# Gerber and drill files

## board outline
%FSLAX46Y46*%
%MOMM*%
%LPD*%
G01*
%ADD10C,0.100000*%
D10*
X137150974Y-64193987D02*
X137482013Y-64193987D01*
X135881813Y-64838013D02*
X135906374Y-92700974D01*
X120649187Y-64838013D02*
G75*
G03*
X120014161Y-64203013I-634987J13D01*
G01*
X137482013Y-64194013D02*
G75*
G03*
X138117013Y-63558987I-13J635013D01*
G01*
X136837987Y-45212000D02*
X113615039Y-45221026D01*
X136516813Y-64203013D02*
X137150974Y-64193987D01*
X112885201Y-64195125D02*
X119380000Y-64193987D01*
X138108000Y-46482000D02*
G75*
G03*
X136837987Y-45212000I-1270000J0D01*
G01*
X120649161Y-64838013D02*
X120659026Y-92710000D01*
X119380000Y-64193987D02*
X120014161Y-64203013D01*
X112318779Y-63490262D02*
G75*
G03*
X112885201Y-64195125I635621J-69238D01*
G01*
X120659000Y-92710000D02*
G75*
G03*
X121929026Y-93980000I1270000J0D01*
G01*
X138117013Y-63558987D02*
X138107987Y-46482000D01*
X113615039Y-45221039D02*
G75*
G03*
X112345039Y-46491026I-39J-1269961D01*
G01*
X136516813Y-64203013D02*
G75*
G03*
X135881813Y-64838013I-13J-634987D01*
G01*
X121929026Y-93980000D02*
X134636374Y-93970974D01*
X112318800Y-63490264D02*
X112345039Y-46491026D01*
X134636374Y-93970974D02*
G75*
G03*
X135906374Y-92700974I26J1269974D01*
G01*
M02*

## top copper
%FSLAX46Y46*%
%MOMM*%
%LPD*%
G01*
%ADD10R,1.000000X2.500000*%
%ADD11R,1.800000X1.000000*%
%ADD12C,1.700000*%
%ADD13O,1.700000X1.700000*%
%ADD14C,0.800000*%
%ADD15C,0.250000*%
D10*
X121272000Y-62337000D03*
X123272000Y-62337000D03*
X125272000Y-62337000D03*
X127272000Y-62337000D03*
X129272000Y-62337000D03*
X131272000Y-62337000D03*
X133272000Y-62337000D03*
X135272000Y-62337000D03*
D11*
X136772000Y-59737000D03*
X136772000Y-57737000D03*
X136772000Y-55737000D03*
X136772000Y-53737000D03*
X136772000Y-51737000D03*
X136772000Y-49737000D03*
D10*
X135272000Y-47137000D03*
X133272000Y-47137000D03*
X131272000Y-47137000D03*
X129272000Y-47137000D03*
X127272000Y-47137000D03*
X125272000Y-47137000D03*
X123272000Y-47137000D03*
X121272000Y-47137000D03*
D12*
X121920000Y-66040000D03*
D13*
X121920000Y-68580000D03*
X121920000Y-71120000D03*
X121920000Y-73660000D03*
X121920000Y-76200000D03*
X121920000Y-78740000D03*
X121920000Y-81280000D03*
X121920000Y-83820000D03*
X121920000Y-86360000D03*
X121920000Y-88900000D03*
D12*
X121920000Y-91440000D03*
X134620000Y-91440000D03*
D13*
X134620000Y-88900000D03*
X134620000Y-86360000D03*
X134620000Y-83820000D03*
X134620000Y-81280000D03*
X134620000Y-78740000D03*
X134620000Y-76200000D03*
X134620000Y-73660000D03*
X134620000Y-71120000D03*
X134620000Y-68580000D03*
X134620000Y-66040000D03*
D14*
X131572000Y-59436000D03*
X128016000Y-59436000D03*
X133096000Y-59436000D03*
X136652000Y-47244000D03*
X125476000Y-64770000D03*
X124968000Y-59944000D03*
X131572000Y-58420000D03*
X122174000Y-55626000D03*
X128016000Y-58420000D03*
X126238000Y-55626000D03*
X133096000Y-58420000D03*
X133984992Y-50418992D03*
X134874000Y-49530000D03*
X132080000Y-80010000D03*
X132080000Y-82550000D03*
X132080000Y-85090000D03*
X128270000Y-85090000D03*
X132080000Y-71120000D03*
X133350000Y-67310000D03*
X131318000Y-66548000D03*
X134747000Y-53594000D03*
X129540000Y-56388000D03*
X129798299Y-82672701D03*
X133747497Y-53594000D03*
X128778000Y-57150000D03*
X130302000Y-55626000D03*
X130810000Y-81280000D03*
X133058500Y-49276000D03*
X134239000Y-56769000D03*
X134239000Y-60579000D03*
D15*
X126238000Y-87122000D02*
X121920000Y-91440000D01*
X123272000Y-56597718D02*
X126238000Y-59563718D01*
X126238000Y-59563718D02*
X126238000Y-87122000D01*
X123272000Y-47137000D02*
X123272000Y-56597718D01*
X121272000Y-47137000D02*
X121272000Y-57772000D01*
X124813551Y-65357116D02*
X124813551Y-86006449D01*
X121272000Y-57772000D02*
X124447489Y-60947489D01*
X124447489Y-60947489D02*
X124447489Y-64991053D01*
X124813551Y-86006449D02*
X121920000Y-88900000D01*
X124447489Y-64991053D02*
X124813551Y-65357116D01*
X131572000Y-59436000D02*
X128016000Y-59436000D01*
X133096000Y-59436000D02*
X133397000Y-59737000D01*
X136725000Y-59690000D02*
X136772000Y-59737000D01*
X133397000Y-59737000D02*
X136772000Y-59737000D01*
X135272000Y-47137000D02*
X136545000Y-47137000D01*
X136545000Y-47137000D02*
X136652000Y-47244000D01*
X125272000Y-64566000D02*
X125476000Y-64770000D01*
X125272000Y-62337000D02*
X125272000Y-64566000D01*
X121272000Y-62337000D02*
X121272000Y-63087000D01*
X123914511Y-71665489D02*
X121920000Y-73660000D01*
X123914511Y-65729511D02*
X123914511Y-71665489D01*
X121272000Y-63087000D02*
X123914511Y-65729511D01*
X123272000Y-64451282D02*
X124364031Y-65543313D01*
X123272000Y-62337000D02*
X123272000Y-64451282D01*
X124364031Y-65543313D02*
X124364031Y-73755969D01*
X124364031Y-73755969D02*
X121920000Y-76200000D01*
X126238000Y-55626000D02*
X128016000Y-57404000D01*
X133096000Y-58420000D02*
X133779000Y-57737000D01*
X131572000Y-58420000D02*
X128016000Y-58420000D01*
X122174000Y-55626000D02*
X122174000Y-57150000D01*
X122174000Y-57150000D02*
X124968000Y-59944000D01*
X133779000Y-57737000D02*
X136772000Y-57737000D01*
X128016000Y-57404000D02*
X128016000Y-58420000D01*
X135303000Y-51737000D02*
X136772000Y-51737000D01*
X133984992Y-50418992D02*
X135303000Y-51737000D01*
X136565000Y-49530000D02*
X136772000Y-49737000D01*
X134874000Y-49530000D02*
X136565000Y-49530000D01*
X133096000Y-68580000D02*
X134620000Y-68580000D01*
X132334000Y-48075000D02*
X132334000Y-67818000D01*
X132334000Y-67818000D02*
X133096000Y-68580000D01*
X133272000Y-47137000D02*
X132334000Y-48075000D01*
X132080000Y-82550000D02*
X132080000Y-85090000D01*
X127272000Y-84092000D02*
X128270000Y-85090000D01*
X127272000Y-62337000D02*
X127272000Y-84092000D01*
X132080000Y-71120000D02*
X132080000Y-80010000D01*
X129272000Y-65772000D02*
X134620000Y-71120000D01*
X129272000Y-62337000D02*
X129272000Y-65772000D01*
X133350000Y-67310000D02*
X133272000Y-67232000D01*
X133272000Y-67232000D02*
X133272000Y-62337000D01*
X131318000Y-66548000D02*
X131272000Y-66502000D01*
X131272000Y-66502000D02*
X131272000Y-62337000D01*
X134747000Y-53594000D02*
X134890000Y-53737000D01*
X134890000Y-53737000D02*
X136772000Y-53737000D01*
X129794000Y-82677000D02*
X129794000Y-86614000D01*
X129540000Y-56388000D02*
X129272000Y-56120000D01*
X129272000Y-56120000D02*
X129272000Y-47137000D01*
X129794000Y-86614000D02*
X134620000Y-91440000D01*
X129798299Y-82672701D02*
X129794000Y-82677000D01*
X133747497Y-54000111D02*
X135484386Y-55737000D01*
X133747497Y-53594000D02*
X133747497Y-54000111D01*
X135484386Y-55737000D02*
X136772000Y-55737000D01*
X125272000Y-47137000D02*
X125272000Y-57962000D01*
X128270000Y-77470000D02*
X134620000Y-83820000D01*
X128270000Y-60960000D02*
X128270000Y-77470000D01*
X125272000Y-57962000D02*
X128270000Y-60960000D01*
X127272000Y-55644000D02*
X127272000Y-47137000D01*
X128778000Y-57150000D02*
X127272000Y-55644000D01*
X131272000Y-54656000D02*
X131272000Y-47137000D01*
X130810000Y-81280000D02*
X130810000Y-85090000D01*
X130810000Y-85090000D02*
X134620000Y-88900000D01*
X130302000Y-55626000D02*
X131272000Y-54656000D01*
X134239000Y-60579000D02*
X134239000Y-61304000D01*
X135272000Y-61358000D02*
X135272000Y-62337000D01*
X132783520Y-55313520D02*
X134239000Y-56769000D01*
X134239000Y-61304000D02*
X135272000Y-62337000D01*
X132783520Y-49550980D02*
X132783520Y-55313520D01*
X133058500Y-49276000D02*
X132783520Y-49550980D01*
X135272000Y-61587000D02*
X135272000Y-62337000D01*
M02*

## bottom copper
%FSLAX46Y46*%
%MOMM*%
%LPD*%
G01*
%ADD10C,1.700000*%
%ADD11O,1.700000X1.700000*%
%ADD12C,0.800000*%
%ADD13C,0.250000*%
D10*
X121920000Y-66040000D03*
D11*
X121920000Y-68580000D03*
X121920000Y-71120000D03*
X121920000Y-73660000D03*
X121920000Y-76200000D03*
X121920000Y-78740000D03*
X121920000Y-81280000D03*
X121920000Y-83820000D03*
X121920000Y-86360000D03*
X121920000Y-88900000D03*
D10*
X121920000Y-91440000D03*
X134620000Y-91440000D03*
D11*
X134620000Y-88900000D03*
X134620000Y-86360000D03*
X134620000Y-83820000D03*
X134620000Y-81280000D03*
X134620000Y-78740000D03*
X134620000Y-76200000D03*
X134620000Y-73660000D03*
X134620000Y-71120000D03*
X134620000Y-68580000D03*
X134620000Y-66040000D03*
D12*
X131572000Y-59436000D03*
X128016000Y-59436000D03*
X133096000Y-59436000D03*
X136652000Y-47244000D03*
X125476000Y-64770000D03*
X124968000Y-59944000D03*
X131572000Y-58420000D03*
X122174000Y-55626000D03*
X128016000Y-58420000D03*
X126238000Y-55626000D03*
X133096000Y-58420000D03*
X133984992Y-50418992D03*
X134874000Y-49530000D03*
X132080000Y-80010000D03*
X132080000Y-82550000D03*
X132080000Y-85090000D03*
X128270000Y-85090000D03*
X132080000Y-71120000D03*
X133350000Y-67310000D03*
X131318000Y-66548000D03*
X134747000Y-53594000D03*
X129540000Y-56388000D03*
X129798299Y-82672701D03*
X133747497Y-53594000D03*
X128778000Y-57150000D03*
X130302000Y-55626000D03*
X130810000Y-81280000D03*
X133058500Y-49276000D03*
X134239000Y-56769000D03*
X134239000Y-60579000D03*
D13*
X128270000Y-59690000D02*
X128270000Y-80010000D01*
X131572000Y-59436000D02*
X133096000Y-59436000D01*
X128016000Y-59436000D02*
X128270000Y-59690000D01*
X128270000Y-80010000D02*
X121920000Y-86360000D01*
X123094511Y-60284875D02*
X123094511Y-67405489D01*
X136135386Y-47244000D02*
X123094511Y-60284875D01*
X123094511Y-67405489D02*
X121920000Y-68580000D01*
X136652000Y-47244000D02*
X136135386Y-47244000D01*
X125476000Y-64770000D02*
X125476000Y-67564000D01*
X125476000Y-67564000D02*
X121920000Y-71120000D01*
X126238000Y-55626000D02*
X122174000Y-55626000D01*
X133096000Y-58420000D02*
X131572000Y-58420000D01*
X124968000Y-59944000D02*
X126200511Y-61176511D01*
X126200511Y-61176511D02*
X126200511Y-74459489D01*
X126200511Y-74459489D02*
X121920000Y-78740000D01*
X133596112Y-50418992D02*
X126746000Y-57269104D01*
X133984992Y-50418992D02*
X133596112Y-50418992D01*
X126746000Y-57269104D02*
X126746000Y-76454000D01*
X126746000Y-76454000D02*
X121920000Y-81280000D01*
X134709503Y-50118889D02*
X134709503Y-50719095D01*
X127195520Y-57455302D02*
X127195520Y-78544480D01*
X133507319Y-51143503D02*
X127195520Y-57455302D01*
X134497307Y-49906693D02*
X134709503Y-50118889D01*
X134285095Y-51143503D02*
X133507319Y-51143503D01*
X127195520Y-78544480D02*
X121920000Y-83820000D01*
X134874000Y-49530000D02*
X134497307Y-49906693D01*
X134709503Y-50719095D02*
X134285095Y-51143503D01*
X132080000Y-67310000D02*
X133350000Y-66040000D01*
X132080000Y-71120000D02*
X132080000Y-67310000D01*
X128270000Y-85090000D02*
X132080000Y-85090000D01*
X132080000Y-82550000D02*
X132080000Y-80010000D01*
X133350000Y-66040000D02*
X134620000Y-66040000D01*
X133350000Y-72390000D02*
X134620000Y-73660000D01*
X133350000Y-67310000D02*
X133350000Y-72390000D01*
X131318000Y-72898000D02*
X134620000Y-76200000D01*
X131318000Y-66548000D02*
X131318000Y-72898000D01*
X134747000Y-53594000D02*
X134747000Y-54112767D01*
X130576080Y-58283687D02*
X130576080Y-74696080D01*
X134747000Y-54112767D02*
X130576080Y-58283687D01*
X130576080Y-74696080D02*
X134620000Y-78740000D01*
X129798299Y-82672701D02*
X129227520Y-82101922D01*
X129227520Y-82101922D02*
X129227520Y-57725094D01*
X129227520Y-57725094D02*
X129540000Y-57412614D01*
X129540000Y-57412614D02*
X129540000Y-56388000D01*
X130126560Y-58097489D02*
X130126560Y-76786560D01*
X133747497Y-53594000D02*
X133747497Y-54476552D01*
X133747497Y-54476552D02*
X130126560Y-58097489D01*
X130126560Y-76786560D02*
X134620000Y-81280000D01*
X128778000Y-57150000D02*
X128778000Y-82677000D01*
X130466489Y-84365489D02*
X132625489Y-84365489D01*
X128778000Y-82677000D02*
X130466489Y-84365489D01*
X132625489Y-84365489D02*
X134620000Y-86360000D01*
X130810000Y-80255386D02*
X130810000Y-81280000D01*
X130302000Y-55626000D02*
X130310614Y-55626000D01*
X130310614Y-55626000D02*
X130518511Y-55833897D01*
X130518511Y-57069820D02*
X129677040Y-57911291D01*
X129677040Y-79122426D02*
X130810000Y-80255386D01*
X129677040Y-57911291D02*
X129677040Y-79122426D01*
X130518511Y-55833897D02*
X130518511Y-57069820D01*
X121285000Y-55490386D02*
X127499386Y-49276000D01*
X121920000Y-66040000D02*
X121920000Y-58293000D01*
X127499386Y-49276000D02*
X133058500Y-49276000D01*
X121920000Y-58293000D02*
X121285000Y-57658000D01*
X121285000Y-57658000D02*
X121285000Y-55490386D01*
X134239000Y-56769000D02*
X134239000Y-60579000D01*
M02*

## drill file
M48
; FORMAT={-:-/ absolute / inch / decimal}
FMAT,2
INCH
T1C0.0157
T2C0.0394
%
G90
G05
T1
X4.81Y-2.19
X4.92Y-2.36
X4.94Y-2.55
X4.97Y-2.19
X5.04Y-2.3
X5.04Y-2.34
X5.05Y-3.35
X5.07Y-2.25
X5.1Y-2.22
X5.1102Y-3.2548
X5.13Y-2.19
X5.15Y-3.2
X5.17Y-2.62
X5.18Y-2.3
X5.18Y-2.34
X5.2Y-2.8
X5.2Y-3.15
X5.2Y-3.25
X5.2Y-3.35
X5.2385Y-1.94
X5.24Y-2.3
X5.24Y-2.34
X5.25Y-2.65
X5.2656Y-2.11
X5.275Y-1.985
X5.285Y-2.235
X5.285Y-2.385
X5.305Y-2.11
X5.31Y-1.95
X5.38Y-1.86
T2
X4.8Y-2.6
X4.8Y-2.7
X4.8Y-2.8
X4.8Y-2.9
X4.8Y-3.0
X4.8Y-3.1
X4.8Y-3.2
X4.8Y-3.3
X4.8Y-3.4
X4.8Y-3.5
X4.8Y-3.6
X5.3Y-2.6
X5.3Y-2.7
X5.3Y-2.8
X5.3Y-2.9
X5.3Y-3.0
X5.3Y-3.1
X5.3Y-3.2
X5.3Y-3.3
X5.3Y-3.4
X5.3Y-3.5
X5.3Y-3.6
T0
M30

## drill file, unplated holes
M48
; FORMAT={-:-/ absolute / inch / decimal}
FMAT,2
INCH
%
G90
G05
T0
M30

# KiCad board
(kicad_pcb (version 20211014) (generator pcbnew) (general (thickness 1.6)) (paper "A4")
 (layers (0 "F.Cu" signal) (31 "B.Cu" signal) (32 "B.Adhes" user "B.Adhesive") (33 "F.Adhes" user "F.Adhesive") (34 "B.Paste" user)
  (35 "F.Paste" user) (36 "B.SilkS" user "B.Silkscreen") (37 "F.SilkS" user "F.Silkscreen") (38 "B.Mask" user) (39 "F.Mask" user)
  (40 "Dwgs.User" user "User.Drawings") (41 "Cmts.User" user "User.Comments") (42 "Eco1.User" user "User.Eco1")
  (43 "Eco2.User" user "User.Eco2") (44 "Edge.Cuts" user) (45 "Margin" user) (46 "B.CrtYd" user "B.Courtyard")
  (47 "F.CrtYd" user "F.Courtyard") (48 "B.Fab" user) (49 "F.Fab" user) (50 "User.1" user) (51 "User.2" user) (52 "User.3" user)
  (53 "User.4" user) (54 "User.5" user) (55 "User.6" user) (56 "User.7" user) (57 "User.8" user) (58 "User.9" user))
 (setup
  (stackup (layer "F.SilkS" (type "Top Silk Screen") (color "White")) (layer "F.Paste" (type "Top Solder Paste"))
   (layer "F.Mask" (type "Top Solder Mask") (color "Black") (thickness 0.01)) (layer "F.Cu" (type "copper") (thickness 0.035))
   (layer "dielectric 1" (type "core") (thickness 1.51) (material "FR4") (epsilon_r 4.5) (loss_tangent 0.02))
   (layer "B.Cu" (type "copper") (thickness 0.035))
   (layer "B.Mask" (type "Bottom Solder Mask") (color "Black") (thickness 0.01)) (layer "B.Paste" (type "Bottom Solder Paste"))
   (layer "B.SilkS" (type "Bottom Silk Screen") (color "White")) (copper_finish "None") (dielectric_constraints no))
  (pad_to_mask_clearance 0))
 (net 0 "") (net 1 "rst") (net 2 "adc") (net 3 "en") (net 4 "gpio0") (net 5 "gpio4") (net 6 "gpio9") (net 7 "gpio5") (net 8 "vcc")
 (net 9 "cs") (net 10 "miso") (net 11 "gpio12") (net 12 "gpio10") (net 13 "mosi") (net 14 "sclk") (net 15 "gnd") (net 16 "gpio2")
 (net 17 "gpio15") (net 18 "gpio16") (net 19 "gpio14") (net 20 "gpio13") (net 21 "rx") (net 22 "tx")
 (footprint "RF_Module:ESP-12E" (layer "F.Cu") (at 124.772 54.737 90)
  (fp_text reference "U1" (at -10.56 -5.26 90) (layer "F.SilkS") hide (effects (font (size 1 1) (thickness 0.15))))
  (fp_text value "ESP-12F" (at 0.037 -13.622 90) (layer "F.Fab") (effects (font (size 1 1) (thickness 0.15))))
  (pad "1" smd rect (at -7.6 -3.5 90) (size 2.5 1) (layers "F.Cu" "F.Paste" "F.Mask") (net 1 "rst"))
  (pad "2" smd rect (at -7.6 -1.5 90) (size 2.5 1) (layers "F.Cu" "F.Paste" "F.Mask") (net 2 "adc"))
  (pad "3" smd rect (at -7.6 0.5 90) (size 2.5 1) (layers "F.Cu" "F.Paste" "F.Mask") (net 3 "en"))
  (pad "4" smd rect (at -7.6 2.5 90) (size 2.5 1) (layers "F.Cu" "F.Paste" "F.Mask") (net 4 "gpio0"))
  (pad "5" smd rect (at -7.6 4.5 90) (size 2.5 1) (layers "F.Cu" "F.Paste" "F.Mask") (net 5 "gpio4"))
  (pad "6" smd rect (at -7.6 6.5 90) (size 2.5 1) (layers "F.Cu" "F.Paste" "F.Mask") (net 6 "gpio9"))
  (pad "7" smd rect (at -7.6 8.5 90) (size 2.5 1) (layers "F.Cu" "F.Paste" "F.Mask") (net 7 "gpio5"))
  (pad "8" smd rect (at -7.6 10.5 90) (size 2.5 1) (layers "F.Cu" "F.Paste" "F.Mask") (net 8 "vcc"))
  (pad "9" smd rect (at -5 12 90) (size 1 1.8) (layers "F.Cu" "F.Paste" "F.Mask") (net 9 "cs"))
  (pad "10" smd rect (at -3 12 90) (size 1 1.8) (layers "F.Cu" "F.Paste" "F.Mask") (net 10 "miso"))
  (pad "11" smd rect (at -1 12 90) (size 1 1.8) (layers "F.Cu" "F.Paste" "F.Mask") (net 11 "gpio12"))
  (pad "12" smd rect (at 1 12 90) (size 1 1.8) (layers "F.Cu" "F.Paste" "F.Mask") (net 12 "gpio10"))
  (pad "13" smd rect (at 3 12 90) (size 1 1.8) (layers "F.Cu" "F.Paste" "F.Mask") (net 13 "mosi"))
  (pad "14" smd rect (at 5 12 90) (size 1 1.8) (layers "F.Cu" "F.Paste" "F.Mask") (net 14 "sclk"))
  (pad "15" smd rect (at 7.6 10.5 90) (size 2.5 1) (layers "F.Cu" "F.Paste" "F.Mask") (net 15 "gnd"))
  (pad "16" smd rect (at 7.6 8.5 90) (size 2.5 1) (layers "F.Cu" "F.Paste" "F.Mask") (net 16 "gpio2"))
  (pad "17" smd rect (at 7.6 6.5 90) (size 2.5 1) (layers "F.Cu" "F.Paste" "F.Mask") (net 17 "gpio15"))
  (pad "18" smd rect (at 7.6 4.5 90) (size 2.5 1) (layers "F.Cu" "F.Paste" "F.Mask") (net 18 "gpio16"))
  (pad "19" smd rect (at 7.6 2.5 90) (size 2.5 1) (layers "F.Cu" "F.Paste" "F.Mask") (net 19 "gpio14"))
  (pad "20" smd rect (at 7.6 0.5 90) (size 2.5 1) (layers "F.Cu" "F.Paste" "F.Mask") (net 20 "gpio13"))
  (pad "21" smd rect (at 7.6 -1.5 90) (size 2.5 1) (layers "F.Cu" "F.Paste" "F.Mask") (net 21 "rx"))
  (pad "22" smd rect (at 7.6 -3.5 90) (size 2.5 1) (layers "F.Cu" "F.Paste" "F.Mask") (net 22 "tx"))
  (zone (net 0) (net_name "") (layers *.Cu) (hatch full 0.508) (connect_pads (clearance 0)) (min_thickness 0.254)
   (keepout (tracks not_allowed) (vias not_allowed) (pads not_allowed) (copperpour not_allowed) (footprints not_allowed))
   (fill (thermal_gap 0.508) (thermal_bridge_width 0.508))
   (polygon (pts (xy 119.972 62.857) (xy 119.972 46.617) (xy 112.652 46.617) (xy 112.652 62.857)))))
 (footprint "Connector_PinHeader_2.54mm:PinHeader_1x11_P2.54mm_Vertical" (layer "B.Cu") (at 121.92 66.04 180)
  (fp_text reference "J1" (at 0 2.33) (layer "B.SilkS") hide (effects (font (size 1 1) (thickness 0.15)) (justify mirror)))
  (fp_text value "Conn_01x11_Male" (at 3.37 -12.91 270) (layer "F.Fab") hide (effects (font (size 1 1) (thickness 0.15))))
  (pad "1" thru_hole circle (at 0 0 180) (size 1.7 1.7) (drill 1) (layers *.Cu *.Mask) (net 8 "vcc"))
  (pad "2" thru_hole oval (at 0 -2.54 180) (size 1.7 1.7) (drill 1) (layers *.Cu *.Mask) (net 15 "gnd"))
  (pad "3" thru_hole oval (at 0 -5.08 180) (size 1.7 1.7) (drill 1) (layers *.Cu *.Mask) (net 3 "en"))
  (pad "4" thru_hole oval (at 0 -7.62 180) (size 1.7 1.7) (drill 1) (layers *.Cu *.Mask) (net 1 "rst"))
  (pad "5" thru_hole oval (at 0 -10.16 180) (size 1.7 1.7) (drill 1) (layers *.Cu *.Mask) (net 2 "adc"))
  (pad "6" thru_hole oval (at 0 -12.7 180) (size 1.7 1.7) (drill 1) (layers *.Cu *.Mask) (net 10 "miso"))
  (pad "7" thru_hole oval (at 0 -15.24 180) (size 1.7 1.7) (drill 1) (layers *.Cu *.Mask) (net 13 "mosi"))
  (pad "8" thru_hole oval (at 0 -17.78 180) (size 1.7 1.7) (drill 1) (layers *.Cu *.Mask) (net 14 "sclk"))
  (pad "9" thru_hole oval (at 0 -20.32 180) (size 1.7 1.7) (drill 1) (layers *.Cu *.Mask) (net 9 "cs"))
  (pad "10" thru_hole oval (at 0 -22.86 180) (size 1.7 1.7) (drill 1) (layers *.Cu *.Mask) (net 22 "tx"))
  (pad "11" thru_hole circle (at 0 -25.4 180) (size 1.7 1.7) (drill 1) (layers *.Cu *.Mask) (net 21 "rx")))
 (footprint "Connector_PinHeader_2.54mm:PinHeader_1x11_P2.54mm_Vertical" (layer "B.Cu") (at 134.62 91.44)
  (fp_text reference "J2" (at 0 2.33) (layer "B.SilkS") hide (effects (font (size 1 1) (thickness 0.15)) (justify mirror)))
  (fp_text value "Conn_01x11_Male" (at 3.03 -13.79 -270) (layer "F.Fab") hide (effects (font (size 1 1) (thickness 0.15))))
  (pad "1" thru_hole circle (at 0 0) (size 1.7 1.7) (drill 1) (layers *.Cu *.Mask "B.SilkS") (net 18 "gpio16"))
  (pad "2" thru_hole oval (at 0 -2.54) (size 1.7 1.7) (drill 1) (layers *.Cu *.Mask) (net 17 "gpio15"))
  (pad "3" thru_hole oval (at 0 -5.08) (size 1.7 1.7) (drill 1) (layers *.Cu *.Mask) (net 19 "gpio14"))
  (pad "4" thru_hole oval (at 0 -7.62) (size 1.7 1.7) (drill 1) (layers *.Cu *.Mask) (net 20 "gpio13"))
  (pad "5" thru_hole oval (at 0 -10.16) (size 1.7 1.7) (drill 1) (layers *.Cu *.Mask) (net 11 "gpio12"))
  (pad "6" thru_hole oval (at 0 -12.7) (size 1.7 1.7) (drill 1) (layers *.Cu *.Mask) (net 12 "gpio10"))
  (pad "7" thru_hole oval (at 0 -15.24) (size 1.7 1.7) (drill 1) (layers *.Cu *.Mask) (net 6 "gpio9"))
  (pad "8" thru_hole oval (at 0 -17.78) (size 1.7 1.7) (drill 1) (layers *.Cu *.Mask) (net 7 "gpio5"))
  (pad "9" thru_hole oval (at 0 -20.32) (size 1.7 1.7) (drill 1) (layers *.Cu *.Mask) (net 5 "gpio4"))
  (pad "10" thru_hole oval (at 0 -22.86) (size 1.7 1.7) (drill 1) (layers *.Cu *.Mask) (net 16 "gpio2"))
  (pad "11" thru_hole oval (at 0 -25.4) (size 1.7 1.7) (drill 1) (layers *.Cu *.Mask) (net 4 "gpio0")))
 (gr_line (start 137.150974 64.193987) (end 137.482013 64.193987) (layer "Edge.Cuts") (width 0.1))
 (gr_line (start 135.881813 64.838013) (end 135.906374 92.700974) (layer "Edge.Cuts") (width 0.1))
 (gr_arc (start 120.014161 64.203013) (mid 120.463174 64.389) (end 120.649161 64.838013) (layer "Edge.Cuts") (width 0.1))
 (gr_arc (start 138.117013 63.558987) (mid 137.931026 64.008) (end 137.482013 64.193987) (layer "Edge.Cuts") (width 0.1))
 (gr_line (start 136.837987 45.212) (end 113.615039 45.221026) (layer "Edge.Cuts") (width 0.1))
 (gr_line (start 136.516813 64.203013) (end 137.150974 64.193987) (layer "Edge.Cuts") (width 0.1))
 (gr_line (start 112.885201 64.195125) (end 119.38 64.193987) (layer "Edge.Cuts") (width 0.1))
 (gr_arc (start 136.837987 45.212) (mid 137.736013 45.583974) (end 138.107987 46.482) (layer "Edge.Cuts") (width 0.1))
 (gr_line (start 120.649161 64.838013) (end 120.659026 92.71) (layer "Edge.Cuts") (width 0.1))
 (gr_line (start 119.38 64.193987) (end 120.014161 64.203013) (layer "Edge.Cuts") (width 0.1))
 (gr_arc (start 112.885201 64.195125) (mid 112.456019 63.96) (end 112.3188 63.490264) (layer "Edge.Cuts") (width 0.1))
 (gr_arc (start 121.929026 93.98) (mid 121.031 93.608026) (end 120.659026 92.71) (layer "Edge.Cuts") (width 0.1))
 (gr_line (start 138.117013 63.558987) (end 138.107987 46.482) (layer "Edge.Cuts") (width 0.1))
 (gr_arc (start 112.345039 46.491026) (mid 112.717013 45.593) (end 113.615039 45.221026) (layer "Edge.Cuts") (width 0.1))
 (gr_arc (start 135.881813 64.838013) (mid 136.0678 64.389) (end 136.516813 64.203013) (layer "Edge.Cuts") (width 0.1))
 (gr_line (start 121.929026 93.98) (end 134.636374 93.970974) (layer "Edge.Cuts") (width 0.1))
 (gr_line (start 112.3188 63.490264) (end 112.345039 46.491026) (layer "Edge.Cuts") (width 0.1))
 (gr_arc (start 135.906374 92.700974) (mid 135.5344 93.599) (end 134.636374 93.970974) (layer "Edge.Cuts") (width 0.1))
 (segment (start 126.238 87.122) (end 121.92 91.44) (width 0.25) (layer "F.Cu") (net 21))
 (segment (start 123.272 56.597718) (end 126.238 59.563718) (width 0.25) (layer "F.Cu") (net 21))
 (segment (start 126.238 59.563718) (end 126.238 87.122) (width 0.25) (layer "F.Cu") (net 21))
 (segment (start 123.272 47.137) (end 123.272 56.597718) (width 0.25) (layer "F.Cu") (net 21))
 (segment (start 121.272 47.137) (end 121.272 57.772) (width 0.25) (layer "F.Cu") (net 22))
 (segment (start 124.813551 65.357116) (end 124.813551 86.006449) (width 0.25) (layer "F.Cu") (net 22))
 (segment (start 121.272 57.772) (end 124.447489 60.947489) (width 0.25) (layer "F.Cu") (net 22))
 (segment (start 124.447489 60.947489) (end 124.447489 64.991053) (width 0.25) (layer "F.Cu") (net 22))
 (segment (start 124.813551 86.006449) (end 121.92 88.9) (width 0.25) (layer "F.Cu") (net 22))
 (segment (start 124.447489 64.991053) (end 124.813551 65.357116) (width 0.25) (layer "F.Cu") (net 22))
 (segment (start 131.572 59.436) (end 128.016 59.436) (width 0.25) (layer "F.Cu") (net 9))
 (segment (start 133.096 59.436) (end 133.397 59.737) (width 0.25) (layer "F.Cu") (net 9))
 (segment (start 136.725 59.69) (end 136.772 59.737) (width 0.25) (layer "F.Cu") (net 9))
 (segment (start 133.397 59.737) (end 136.772 59.737) (width 0.25) (layer "F.Cu") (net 9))
 (via (at 131.572 59.436) (size 0.8) (drill 0.4) (layers "F.Cu" "B.Cu") (free) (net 9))
 (via (at 128.016 59.436) (size 0.8) (drill 0.4) (layers "F.Cu" "B.Cu") (free) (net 9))
 (via (at 133.096 59.436) (size 0.8) (drill 0.4) (layers "F.Cu" "B.Cu") (free) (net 9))
 (segment (start 128.27 59.69) (end 128.27 80.01) (width 0.25) (layer "B.Cu") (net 9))
 (segment (start 131.572 59.436) (end 133.096 59.436) (width 0.25) (layer "B.Cu") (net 9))
 (segment (start 128.016 59.436) (end 128.27 59.69) (width 0.25) (layer "B.Cu") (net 9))
 (segment (start 128.27 80.01) (end 121.92 86.36) (width 0.25) (layer "B.Cu") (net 9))
 (segment (start 135.272 47.137) (end 136.545 47.137) (width 0.25) (layer "F.Cu") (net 15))
 (segment (start 136.545 47.137) (end 136.652 47.244) (width 0.25) (layer "F.Cu") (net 15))
 (via (at 136.652 47.244) (size 0.8) (drill 0.4) (layers "F.Cu" "B.Cu") (free) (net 15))
 (segment (start 123.094511 60.284875) (end 123.094511 67.405489) (width 0.25) (layer "B.Cu") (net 15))
 (segment (start 136.135386 47.244) (end 123.094511 60.284875) (width 0.25) (layer "B.Cu") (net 15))
 (segment (start 123.094511 67.405489) (end 121.92 68.58) (width 0.25) (layer "B.Cu") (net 15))
 (segment (start 136.652 47.244) (end 136.135386 47.244) (width 0.25) (layer "B.Cu") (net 15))
 (segment (start 125.272 64.566) (end 125.476 64.77) (width 0.25) (layer "F.Cu") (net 3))
 (segment (start 125.272 62.337) (end 125.272 64.566) (width 0.25) (layer "F.Cu") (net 3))
 (via (at 125.476 64.77) (size 0.8) (drill 0.4) (layers "F.Cu" "B.Cu") (free) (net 3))
 (segment (start 125.476 64.77) (end 125.476 67.564) (width 0.25) (layer "B.Cu") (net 3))
 (segment (start 125.476 67.564) (end 121.92 71.12) (width 0.25) (layer "B.Cu") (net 3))
 (segment (start 121.272 62.337) (end 121.272 63.087) (width 0.25) (layer "F.Cu") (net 1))
 (segment (start 123.914511 71.665489) (end 121.92 73.66) (width 0.25) (layer "F.Cu") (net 1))
 (segment (start 123.914511 65.729511) (end 123.914511 71.665489) (width 0.25) (layer "F.Cu") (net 1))
 (segment (start 121.272 63.087) (end 123.914511 65.729511) (width 0.25) (layer "F.Cu") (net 1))
 (segment (start 123.272 64.451282) (end 124.364031 65.543313) (width 0.25) (layer "F.Cu") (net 2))
 (segment (start 123.272 62.337) (end 123.272 64.451282) (width 0.25) (layer "F.Cu") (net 2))
 (segment (start 124.364031 65.543313) (end 124.364031 73.755969) (width 0.25) (layer "F.Cu") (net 2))
 (segment (start 124.364031 73.755969) (end 121.92 76.2) (width 0.25) (layer "F.Cu") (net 2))
 (segment (start 126.238 55.626) (end 128.016 57.404) (width 0.25) (layer "F.Cu") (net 10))
 (segment (start 133.096 58.42) (end 133.779 57.737) (width 0.25) (layer "F.Cu") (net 10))
 (segment (start 131.572 58.42) (end 128.016 58.42) (width 0.25) (layer "F.Cu") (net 10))
 (segment (start 122.174 55.626) (end 122.174 57.15) (width 0.25) (layer "F.Cu") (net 10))
 (segment (start 122.174 57.15) (end 124.968 59.944) (width 0.25) (layer "F.Cu") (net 10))
 (segment (start 133.779 57.737) (end 136.772 57.737) (width 0.25) (layer "F.Cu") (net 10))
 (segment (start 128.016 57.404) (end 128.016 58.42) (width 0.25) (layer "F.Cu") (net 10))
 (via (at 124.968 59.944) (size 0.8) (drill 0.4) (layers "F.Cu" "B.Cu") (free) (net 10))
 (via (at 131.572 58.42) (size 0.8) (drill 0.4) (layers "F.Cu" "B.Cu") (free) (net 10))
 (via (at 122.174 55.626) (size 0.8) (drill 0.4) (layers "F.Cu" "B.Cu") (free) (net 10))
 (via (at 128.016 58.42) (size 0.8) (drill 0.4) (layers "F.Cu" "B.Cu") (free) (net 10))
 (via (at 126.238 55.626) (size 0.8) (drill 0.4) (layers "F.Cu" "B.Cu") (free) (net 10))
 (via (at 133.096 58.42) (size 0.8) (drill 0.4) (layers "F.Cu" "B.Cu") (free) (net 10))
 (segment (start 126.238 55.626) (end 122.174 55.626) (width 0.25) (layer "B.Cu") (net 10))
 (segment (start 133.096 58.42) (end 131.572 58.42) (width 0.25) (layer "B.Cu") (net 10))
 (segment (start 124.968 59.944) (end 126.200511 61.176511) (width 0.25) (layer "B.Cu") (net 10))
 (segment (start 126.200511 61.176511) (end 126.200511 74.459489) (width 0.25) (layer "B.Cu") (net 10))
 (segment (start 126.200511 74.459489) (end 121.92 78.74) (width 0.25) (layer "B.Cu") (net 10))
 (segment (start 135.303 51.737) (end 136.772 51.737) (width 0.25) (layer "F.Cu") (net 13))
 (segment (start 133.984992 50.418992) (end 135.303 51.737) (width 0.25) (layer "F.Cu") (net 13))
 (via (at 133.984992 50.418992) (size 0.8) (drill 0.4) (layers "F.Cu" "B.Cu") (free) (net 13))
 (segment (start 133.596112 50.418992) (end 126.746 57.269104) (width 0.25) (layer "B.Cu") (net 13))
 (segment (start 133.984992 50.418992) (end 133.596112 50.418992) (width 0.25) (layer "B.Cu") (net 13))
 (segment (start 126.746 57.269104) (end 126.746 76.454) (width 0.25) (layer "B.Cu") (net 13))
 (segment (start 126.746 76.454) (end 121.92 81.28) (width 0.25) (layer "B.Cu") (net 13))
 (segment (start 136.565 49.53) (end 136.772 49.737) (width 0.25) (layer "F.Cu") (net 14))
 (segment (start 134.874 49.53) (end 136.565 49.53) (width 0.25) (layer "F.Cu") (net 14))
 (via (at 134.874 49.53) (size 0.8) (drill 0.4) (layers "F.Cu" "B.Cu") (free) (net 14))
 (segment (start 134.709503 50.118889) (end 134.709503 50.719095) (width 0.25) (layer "B.Cu") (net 14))
 (segment (start 127.19552 57.455302) (end 127.19552 78.54448) (width 0.25) (layer "B.Cu") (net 14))
 (segment (start 133.507319 51.143503) (end 127.19552 57.455302) (width 0.25) (layer "B.Cu") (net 14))
 (segment (start 134.497307 49.906693) (end 134.709503 50.118889) (width 0.25) (layer "B.Cu") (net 14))
 (segment (start 134.285095 51.143503) (end 133.507319 51.143503) (width 0.25) (layer "B.Cu") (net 14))
 (segment (start 127.19552 78.54448) (end 121.92 83.82) (width 0.25) (layer "B.Cu") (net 14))
 (segment (start 134.874 49.53) (end 134.497307 49.906693) (width 0.25) (layer "B.Cu") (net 14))
 (segment (start 134.709503 50.719095) (end 134.285095 51.143503) (width 0.25) (layer "B.Cu") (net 14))
 (segment (start 133.096 68.58) (end 134.62 68.58) (width 0.25) (layer "F.Cu") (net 16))
 (segment (start 132.334 48.075) (end 132.334 67.818) (width 0.25) (layer "F.Cu") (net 16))
 (segment (start 132.334 67.818) (end 133.096 68.58) (width 0.25) (layer "F.Cu") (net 16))
 (segment (start 133.272 47.137) (end 132.334 48.075) (width 0.25) (layer "F.Cu") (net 16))
 (segment (start 132.08 82.55) (end 132.08 85.09) (width 0.25) (layer "F.Cu") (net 4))
 (segment (start 127.272 84.092) (end 128.27 85.09) (width 0.25) (layer "F.Cu") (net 4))
 (segment (start 127.272 62.337) (end 127.272 84.092) (width 0.25) (layer "F.Cu") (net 4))
 (segment (start 132.08 71.12) (end 132.08 80.01) (width 0.25) (layer "F.Cu") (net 4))
 (via (at 132.08 80.01) (size 0.8) (drill 0.4) (layers "F.Cu" "B.Cu") (free) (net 4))
 (via (at 132.08 82.55) (size 0.8) (drill 0.4) (layers "F.Cu" "B.Cu") (free) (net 4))
 (via (at 132.08 85.09) (size 0.8) (drill 0.4) (layers "F.Cu" "B.Cu") (free) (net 4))
 (via (at 128.27 85.09) (size 0.8) (drill 0.4) (layers "F.Cu" "B.Cu") (free) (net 4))
 (via (at 132.08 71.12) (size 0.8) (drill 0.4) (layers "F.Cu" "B.Cu") (free) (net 4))
 (segment (start 132.08 67.31) (end 133.35 66.04) (width 0.25) (layer "B.Cu") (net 4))
 (segment (start 132.08 71.12) (end 132.08 67.31) (width 0.25) (layer "B.Cu") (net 4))
 (segment (start 128.27 85.09) (end 132.08 85.09) (width 0.25) (layer "B.Cu") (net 4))
 (segment (start 132.08 82.55) (end 132.08 80.01) (width 0.25) (layer "B.Cu") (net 4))
 (segment (start 133.35 66.04) (end 134.62 66.04) (width 0.25) (layer "B.Cu") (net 4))
 (segment (start 129.272 65.772) (end 134.62 71.12) (width 0.25) (layer "F.Cu") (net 5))
 (segment (start 129.272 62.337) (end 129.272 65.772) (width 0.25) (layer "F.Cu") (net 5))
 (segment (start 133.35 67.31) (end 133.272 67.232) (width 0.25) (layer "F.Cu") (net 7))
 (segment (start 133.272 67.232) (end 133.272 62.337) (width 0.25) (layer "F.Cu") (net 7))
 (via (at 133.35 67.31) (size 0.8) (drill 0.4) (layers "F.Cu" "B.Cu") (free) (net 7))
 (segment (start 133.35 72.39) (end 134.62 73.66) (width 0.25) (layer "B.Cu") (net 7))
 (segment (start 133.35 67.31) (end 133.35 72.39) (width 0.25) (layer "B.Cu") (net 7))
 (segment (start 131.318 66.548) (end 131.272 66.502) (width 0.25) (layer "F.Cu") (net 6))
 (segment (start 131.272 66.502) (end 131.272 62.337) (width 0.25) (layer "F.Cu") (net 6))
 (via (at 131.318 66.548) (size 0.8) (drill 0.4) (layers "F.Cu" "B.Cu") (free) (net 6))
 (segment (start 131.318 72.898) (end 134.62 76.2) (width 0.25) (layer "B.Cu") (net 6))
 (segment (start 131.318 66.548) (end 131.318 72.898) (width 0.25) (layer "B.Cu") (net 6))
 (segment (start 134.747 53.594) (end 134.89 53.737) (width 0.25) (layer "F.Cu") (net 12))
 (segment (start 134.89 53.737) (end 136.772 53.737) (width 0.25) (layer "F.Cu") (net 12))
 (via (at 134.747 53.594) (size 0.8) (drill 0.4) (layers "F.Cu" "B.Cu") (free) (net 12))
 (segment (start 134.747 53.594) (end 134.747 54.112767) (width 0.25) (layer "B.Cu") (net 12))
 (segment (start 130.57608 58.283687) (end 130.57608 74.69608) (width 0.25) (layer "B.Cu") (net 12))
 (segment (start 134.747 54.112767) (end 130.57608 58.283687) (width 0.25) (layer "B.Cu") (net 12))
 (segment (start 130.57608 74.69608) (end 134.62 78.74) (width 0.25) (layer "B.Cu") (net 12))
 (segment (start 129.794 82.677) (end 129.794 86.614) (width 0.25) (layer "F.Cu") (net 18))
 (segment (start 129.54 56.388) (end 129.272 56.12) (width 0.25) (layer "F.Cu") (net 18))
 (segment (start 129.272 56.12) (end 129.272 47.137) (width 0.25) (layer "F.Cu") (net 18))
 (segment (start 129.794 86.614) (end 134.62 91.44) (width 0.25) (layer "F.Cu") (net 18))
 (segment (start 129.798299 82.672701) (end 129.794 82.677) (width 0.25) (layer "F.Cu") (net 18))
 (via (at 129.54 56.388) (size 0.8) (drill 0.4) (layers "F.Cu" "B.Cu") (free) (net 18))
 (via (at 129.798299 82.672701) (size 0.8) (drill 0.4) (layers "F.Cu" "B.Cu") (free) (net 18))
 (segment (start 129.798299 82.672701) (end 129.22752 82.101922) (width 0.25) (layer "B.Cu") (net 18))
 (segment (start 129.22752 82.101922) (end 129.22752 57.725094) (width 0.25) (layer "B.Cu") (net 18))
 (segment (start 129.22752 57.725094) (end 129.54 57.412614) (width 0.25) (layer "B.Cu") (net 18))
 (segment (start 129.54 57.412614) (end 129.54 56.388) (width 0.25) (layer "B.Cu") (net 18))
 (segment (start 133.747497 54.000111) (end 135.484386 55.737) (width 0.25) (layer "F.Cu") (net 11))
 (segment (start 133.747497 53.594) (end 133.747497 54.000111) (width 0.25) (layer "F.Cu") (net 11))
 (segment (start 135.484386 55.737) (end 136.772 55.737) (width 0.25) (layer "F.Cu") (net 11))
 (via (at 133.747497 53.594) (size 0.8) (drill 0.4) (layers "F.Cu" "B.Cu") (free) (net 11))
 (segment (start 130.12656 58.097489) (end 130.12656 76.78656) (width 0.25) (layer "B.Cu") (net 11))
 (segment (start 133.747497 53.594) (end 133.747497 54.476552) (width 0.25) (layer "B.Cu") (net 11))
 (segment (start 133.747497 54.476552) (end 130.12656 58.097489) (width 0.25) (layer "B.Cu") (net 11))
 (segment (start 130.12656 76.78656) (end 134.62 81.28) (width 0.25) (layer "B.Cu") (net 11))
 (segment (start 125.272 47.137) (end 125.272 57.962) (width 0.25) (layer "F.Cu") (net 20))
 (segment (start 128.27 77.47) (end 134.62 83.82) (width 0.25) (layer "F.Cu") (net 20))
 (segment (start 128.27 60.96) (end 128.27 77.47) (width 0.25) (layer "F.Cu") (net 20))
 (segment (start 125.272 57.962) (end 128.27 60.96) (width 0.25) (layer "F.Cu") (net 20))
 (segment (start 127.272 55.644) (end 127.272 47.137) (width 0.25) (layer "F.Cu") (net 19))
 (segment (start 128.778 57.15) (end 127.272 55.644) (width 0.25) (layer "F.Cu") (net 19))
 (via (at 128.778 57.15) (size 0.8) (drill 0.4) (layers "F.Cu" "B.Cu") (free) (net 19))
 (segment (start 128.778 57.15) (end 128.778 82.677) (width 0.25) (layer "B.Cu") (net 19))
 (segment (start 130.466489 84.365489) (end 132.625489 84.365489) (width 0.25) (layer "B.Cu") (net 19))
 (segment (start 128.778 82.677) (end 130.466489 84.365489) (width 0.25) (layer "B.Cu") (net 19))
 (segment (start 132.625489 84.365489) (end 134.62 86.36) (width 0.25) (layer "B.Cu") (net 19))
 (segment (start 131.272 54.656) (end 131.272 47.137) (width 0.25) (layer "F.Cu") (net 17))
 (segment (start 130.81 81.28) (end 130.81 85.09) (width 0.25) (layer "F.Cu") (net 17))
 (segment (start 130.81 85.09) (end 134.62 88.9) (width 0.25) (layer "F.Cu") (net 17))
 (segment (start 130.302 55.626) (end 131.272 54.656) (width 0.25) (layer "F.Cu") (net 17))
 (via (at 130.302 55.626) (size 0.8) (drill 0.4) (layers "F.Cu" "B.Cu") (free) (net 17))
 (via (at 130.81 81.28) (size 0.8) (drill 0.4) (layers "F.Cu" "B.Cu") (free) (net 17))
 (segment (start 130.81 80.255386) (end 130.81 81.28) (width 0.25) (layer "B.Cu") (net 17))
 (segment (start 130.302 55.626) (end 130.310614 55.626) (width 0.25) (layer "B.Cu") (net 17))
 (segment (start 130.310614 55.626) (end 130.518511 55.833897) (width 0.25) (layer "B.Cu") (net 17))
 (segment (start 130.518511 57.06982) (end 129.67704 57.911291) (width 0.25) (layer "B.Cu") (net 17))
 (segment (start 129.67704 79.122426) (end 130.81 80.255386) (width 0.25) (layer "B.Cu") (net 17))
 (segment (start 129.67704 57.911291) (end 129.67704 79.122426) (width 0.25) (layer "B.Cu") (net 17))
 (segment (start 130.518511 55.833897) (end 130.518511 57.06982) (width 0.25) (layer "B.Cu") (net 17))
 (segment (start 134.239 60.579) (end 134.239 61.304) (width 0.25) (layer "F.Cu") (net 8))
 (segment (start 135.272 61.358) (end 135.272 62.337) (width 0.25) (layer "F.Cu") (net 8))
 (segment (start 132.78352 55.31352) (end 134.239 56.769) (width 0.25) (layer "F.Cu") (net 8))
 (segment (start 134.239 61.304) (end 135.272 62.337) (width 0.25) (layer "F.Cu") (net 8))
 (segment (start 132.78352 49.55098) (end 132.78352 55.31352) (width 0.25) (layer "F.Cu") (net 8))
 (segment (start 133.0585 49.276) (end 132.78352 49.55098) (width 0.25) (layer "F.Cu") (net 8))
 (segment (start 135.272 61.587) (end 135.272 62.337) (width 0.25) (layer "F.Cu") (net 8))
 (via (at 133.0585 49.276) (size 0.8) (drill 0.4) (layers "F.Cu" "B.Cu") (free) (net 8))
 (via (at 134.239 56.769) (size 0.8) (drill 0.4) (layers "F.Cu" "B.Cu") (free) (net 8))
 (via (at 134.239 60.579) (size 0.8) (drill 0.4) (layers "F.Cu" "B.Cu") (free) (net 8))
 (segment (start 121.285 55.490386) (end 127.499386 49.276) (width 0.25) (layer "B.Cu") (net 8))
 (segment (start 121.92 66.04) (end 121.92 58.293) (width 0.25) (layer "B.Cu") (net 8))
 (segment (start 127.499386 49.276) (end 133.0585 49.276) (width 0.25) (layer "B.Cu") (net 8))
 (segment (start 121.92 58.293) (end 121.285 57.658) (width 0.25) (layer "B.Cu") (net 8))
 (segment (start 121.285 57.658) (end 121.285 55.490386) (width 0.25) (layer "B.Cu") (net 8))
 (segment (start 134.239 56.769) (end 134.239 60.579) (width 0.25) (layer "B.Cu") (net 8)))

